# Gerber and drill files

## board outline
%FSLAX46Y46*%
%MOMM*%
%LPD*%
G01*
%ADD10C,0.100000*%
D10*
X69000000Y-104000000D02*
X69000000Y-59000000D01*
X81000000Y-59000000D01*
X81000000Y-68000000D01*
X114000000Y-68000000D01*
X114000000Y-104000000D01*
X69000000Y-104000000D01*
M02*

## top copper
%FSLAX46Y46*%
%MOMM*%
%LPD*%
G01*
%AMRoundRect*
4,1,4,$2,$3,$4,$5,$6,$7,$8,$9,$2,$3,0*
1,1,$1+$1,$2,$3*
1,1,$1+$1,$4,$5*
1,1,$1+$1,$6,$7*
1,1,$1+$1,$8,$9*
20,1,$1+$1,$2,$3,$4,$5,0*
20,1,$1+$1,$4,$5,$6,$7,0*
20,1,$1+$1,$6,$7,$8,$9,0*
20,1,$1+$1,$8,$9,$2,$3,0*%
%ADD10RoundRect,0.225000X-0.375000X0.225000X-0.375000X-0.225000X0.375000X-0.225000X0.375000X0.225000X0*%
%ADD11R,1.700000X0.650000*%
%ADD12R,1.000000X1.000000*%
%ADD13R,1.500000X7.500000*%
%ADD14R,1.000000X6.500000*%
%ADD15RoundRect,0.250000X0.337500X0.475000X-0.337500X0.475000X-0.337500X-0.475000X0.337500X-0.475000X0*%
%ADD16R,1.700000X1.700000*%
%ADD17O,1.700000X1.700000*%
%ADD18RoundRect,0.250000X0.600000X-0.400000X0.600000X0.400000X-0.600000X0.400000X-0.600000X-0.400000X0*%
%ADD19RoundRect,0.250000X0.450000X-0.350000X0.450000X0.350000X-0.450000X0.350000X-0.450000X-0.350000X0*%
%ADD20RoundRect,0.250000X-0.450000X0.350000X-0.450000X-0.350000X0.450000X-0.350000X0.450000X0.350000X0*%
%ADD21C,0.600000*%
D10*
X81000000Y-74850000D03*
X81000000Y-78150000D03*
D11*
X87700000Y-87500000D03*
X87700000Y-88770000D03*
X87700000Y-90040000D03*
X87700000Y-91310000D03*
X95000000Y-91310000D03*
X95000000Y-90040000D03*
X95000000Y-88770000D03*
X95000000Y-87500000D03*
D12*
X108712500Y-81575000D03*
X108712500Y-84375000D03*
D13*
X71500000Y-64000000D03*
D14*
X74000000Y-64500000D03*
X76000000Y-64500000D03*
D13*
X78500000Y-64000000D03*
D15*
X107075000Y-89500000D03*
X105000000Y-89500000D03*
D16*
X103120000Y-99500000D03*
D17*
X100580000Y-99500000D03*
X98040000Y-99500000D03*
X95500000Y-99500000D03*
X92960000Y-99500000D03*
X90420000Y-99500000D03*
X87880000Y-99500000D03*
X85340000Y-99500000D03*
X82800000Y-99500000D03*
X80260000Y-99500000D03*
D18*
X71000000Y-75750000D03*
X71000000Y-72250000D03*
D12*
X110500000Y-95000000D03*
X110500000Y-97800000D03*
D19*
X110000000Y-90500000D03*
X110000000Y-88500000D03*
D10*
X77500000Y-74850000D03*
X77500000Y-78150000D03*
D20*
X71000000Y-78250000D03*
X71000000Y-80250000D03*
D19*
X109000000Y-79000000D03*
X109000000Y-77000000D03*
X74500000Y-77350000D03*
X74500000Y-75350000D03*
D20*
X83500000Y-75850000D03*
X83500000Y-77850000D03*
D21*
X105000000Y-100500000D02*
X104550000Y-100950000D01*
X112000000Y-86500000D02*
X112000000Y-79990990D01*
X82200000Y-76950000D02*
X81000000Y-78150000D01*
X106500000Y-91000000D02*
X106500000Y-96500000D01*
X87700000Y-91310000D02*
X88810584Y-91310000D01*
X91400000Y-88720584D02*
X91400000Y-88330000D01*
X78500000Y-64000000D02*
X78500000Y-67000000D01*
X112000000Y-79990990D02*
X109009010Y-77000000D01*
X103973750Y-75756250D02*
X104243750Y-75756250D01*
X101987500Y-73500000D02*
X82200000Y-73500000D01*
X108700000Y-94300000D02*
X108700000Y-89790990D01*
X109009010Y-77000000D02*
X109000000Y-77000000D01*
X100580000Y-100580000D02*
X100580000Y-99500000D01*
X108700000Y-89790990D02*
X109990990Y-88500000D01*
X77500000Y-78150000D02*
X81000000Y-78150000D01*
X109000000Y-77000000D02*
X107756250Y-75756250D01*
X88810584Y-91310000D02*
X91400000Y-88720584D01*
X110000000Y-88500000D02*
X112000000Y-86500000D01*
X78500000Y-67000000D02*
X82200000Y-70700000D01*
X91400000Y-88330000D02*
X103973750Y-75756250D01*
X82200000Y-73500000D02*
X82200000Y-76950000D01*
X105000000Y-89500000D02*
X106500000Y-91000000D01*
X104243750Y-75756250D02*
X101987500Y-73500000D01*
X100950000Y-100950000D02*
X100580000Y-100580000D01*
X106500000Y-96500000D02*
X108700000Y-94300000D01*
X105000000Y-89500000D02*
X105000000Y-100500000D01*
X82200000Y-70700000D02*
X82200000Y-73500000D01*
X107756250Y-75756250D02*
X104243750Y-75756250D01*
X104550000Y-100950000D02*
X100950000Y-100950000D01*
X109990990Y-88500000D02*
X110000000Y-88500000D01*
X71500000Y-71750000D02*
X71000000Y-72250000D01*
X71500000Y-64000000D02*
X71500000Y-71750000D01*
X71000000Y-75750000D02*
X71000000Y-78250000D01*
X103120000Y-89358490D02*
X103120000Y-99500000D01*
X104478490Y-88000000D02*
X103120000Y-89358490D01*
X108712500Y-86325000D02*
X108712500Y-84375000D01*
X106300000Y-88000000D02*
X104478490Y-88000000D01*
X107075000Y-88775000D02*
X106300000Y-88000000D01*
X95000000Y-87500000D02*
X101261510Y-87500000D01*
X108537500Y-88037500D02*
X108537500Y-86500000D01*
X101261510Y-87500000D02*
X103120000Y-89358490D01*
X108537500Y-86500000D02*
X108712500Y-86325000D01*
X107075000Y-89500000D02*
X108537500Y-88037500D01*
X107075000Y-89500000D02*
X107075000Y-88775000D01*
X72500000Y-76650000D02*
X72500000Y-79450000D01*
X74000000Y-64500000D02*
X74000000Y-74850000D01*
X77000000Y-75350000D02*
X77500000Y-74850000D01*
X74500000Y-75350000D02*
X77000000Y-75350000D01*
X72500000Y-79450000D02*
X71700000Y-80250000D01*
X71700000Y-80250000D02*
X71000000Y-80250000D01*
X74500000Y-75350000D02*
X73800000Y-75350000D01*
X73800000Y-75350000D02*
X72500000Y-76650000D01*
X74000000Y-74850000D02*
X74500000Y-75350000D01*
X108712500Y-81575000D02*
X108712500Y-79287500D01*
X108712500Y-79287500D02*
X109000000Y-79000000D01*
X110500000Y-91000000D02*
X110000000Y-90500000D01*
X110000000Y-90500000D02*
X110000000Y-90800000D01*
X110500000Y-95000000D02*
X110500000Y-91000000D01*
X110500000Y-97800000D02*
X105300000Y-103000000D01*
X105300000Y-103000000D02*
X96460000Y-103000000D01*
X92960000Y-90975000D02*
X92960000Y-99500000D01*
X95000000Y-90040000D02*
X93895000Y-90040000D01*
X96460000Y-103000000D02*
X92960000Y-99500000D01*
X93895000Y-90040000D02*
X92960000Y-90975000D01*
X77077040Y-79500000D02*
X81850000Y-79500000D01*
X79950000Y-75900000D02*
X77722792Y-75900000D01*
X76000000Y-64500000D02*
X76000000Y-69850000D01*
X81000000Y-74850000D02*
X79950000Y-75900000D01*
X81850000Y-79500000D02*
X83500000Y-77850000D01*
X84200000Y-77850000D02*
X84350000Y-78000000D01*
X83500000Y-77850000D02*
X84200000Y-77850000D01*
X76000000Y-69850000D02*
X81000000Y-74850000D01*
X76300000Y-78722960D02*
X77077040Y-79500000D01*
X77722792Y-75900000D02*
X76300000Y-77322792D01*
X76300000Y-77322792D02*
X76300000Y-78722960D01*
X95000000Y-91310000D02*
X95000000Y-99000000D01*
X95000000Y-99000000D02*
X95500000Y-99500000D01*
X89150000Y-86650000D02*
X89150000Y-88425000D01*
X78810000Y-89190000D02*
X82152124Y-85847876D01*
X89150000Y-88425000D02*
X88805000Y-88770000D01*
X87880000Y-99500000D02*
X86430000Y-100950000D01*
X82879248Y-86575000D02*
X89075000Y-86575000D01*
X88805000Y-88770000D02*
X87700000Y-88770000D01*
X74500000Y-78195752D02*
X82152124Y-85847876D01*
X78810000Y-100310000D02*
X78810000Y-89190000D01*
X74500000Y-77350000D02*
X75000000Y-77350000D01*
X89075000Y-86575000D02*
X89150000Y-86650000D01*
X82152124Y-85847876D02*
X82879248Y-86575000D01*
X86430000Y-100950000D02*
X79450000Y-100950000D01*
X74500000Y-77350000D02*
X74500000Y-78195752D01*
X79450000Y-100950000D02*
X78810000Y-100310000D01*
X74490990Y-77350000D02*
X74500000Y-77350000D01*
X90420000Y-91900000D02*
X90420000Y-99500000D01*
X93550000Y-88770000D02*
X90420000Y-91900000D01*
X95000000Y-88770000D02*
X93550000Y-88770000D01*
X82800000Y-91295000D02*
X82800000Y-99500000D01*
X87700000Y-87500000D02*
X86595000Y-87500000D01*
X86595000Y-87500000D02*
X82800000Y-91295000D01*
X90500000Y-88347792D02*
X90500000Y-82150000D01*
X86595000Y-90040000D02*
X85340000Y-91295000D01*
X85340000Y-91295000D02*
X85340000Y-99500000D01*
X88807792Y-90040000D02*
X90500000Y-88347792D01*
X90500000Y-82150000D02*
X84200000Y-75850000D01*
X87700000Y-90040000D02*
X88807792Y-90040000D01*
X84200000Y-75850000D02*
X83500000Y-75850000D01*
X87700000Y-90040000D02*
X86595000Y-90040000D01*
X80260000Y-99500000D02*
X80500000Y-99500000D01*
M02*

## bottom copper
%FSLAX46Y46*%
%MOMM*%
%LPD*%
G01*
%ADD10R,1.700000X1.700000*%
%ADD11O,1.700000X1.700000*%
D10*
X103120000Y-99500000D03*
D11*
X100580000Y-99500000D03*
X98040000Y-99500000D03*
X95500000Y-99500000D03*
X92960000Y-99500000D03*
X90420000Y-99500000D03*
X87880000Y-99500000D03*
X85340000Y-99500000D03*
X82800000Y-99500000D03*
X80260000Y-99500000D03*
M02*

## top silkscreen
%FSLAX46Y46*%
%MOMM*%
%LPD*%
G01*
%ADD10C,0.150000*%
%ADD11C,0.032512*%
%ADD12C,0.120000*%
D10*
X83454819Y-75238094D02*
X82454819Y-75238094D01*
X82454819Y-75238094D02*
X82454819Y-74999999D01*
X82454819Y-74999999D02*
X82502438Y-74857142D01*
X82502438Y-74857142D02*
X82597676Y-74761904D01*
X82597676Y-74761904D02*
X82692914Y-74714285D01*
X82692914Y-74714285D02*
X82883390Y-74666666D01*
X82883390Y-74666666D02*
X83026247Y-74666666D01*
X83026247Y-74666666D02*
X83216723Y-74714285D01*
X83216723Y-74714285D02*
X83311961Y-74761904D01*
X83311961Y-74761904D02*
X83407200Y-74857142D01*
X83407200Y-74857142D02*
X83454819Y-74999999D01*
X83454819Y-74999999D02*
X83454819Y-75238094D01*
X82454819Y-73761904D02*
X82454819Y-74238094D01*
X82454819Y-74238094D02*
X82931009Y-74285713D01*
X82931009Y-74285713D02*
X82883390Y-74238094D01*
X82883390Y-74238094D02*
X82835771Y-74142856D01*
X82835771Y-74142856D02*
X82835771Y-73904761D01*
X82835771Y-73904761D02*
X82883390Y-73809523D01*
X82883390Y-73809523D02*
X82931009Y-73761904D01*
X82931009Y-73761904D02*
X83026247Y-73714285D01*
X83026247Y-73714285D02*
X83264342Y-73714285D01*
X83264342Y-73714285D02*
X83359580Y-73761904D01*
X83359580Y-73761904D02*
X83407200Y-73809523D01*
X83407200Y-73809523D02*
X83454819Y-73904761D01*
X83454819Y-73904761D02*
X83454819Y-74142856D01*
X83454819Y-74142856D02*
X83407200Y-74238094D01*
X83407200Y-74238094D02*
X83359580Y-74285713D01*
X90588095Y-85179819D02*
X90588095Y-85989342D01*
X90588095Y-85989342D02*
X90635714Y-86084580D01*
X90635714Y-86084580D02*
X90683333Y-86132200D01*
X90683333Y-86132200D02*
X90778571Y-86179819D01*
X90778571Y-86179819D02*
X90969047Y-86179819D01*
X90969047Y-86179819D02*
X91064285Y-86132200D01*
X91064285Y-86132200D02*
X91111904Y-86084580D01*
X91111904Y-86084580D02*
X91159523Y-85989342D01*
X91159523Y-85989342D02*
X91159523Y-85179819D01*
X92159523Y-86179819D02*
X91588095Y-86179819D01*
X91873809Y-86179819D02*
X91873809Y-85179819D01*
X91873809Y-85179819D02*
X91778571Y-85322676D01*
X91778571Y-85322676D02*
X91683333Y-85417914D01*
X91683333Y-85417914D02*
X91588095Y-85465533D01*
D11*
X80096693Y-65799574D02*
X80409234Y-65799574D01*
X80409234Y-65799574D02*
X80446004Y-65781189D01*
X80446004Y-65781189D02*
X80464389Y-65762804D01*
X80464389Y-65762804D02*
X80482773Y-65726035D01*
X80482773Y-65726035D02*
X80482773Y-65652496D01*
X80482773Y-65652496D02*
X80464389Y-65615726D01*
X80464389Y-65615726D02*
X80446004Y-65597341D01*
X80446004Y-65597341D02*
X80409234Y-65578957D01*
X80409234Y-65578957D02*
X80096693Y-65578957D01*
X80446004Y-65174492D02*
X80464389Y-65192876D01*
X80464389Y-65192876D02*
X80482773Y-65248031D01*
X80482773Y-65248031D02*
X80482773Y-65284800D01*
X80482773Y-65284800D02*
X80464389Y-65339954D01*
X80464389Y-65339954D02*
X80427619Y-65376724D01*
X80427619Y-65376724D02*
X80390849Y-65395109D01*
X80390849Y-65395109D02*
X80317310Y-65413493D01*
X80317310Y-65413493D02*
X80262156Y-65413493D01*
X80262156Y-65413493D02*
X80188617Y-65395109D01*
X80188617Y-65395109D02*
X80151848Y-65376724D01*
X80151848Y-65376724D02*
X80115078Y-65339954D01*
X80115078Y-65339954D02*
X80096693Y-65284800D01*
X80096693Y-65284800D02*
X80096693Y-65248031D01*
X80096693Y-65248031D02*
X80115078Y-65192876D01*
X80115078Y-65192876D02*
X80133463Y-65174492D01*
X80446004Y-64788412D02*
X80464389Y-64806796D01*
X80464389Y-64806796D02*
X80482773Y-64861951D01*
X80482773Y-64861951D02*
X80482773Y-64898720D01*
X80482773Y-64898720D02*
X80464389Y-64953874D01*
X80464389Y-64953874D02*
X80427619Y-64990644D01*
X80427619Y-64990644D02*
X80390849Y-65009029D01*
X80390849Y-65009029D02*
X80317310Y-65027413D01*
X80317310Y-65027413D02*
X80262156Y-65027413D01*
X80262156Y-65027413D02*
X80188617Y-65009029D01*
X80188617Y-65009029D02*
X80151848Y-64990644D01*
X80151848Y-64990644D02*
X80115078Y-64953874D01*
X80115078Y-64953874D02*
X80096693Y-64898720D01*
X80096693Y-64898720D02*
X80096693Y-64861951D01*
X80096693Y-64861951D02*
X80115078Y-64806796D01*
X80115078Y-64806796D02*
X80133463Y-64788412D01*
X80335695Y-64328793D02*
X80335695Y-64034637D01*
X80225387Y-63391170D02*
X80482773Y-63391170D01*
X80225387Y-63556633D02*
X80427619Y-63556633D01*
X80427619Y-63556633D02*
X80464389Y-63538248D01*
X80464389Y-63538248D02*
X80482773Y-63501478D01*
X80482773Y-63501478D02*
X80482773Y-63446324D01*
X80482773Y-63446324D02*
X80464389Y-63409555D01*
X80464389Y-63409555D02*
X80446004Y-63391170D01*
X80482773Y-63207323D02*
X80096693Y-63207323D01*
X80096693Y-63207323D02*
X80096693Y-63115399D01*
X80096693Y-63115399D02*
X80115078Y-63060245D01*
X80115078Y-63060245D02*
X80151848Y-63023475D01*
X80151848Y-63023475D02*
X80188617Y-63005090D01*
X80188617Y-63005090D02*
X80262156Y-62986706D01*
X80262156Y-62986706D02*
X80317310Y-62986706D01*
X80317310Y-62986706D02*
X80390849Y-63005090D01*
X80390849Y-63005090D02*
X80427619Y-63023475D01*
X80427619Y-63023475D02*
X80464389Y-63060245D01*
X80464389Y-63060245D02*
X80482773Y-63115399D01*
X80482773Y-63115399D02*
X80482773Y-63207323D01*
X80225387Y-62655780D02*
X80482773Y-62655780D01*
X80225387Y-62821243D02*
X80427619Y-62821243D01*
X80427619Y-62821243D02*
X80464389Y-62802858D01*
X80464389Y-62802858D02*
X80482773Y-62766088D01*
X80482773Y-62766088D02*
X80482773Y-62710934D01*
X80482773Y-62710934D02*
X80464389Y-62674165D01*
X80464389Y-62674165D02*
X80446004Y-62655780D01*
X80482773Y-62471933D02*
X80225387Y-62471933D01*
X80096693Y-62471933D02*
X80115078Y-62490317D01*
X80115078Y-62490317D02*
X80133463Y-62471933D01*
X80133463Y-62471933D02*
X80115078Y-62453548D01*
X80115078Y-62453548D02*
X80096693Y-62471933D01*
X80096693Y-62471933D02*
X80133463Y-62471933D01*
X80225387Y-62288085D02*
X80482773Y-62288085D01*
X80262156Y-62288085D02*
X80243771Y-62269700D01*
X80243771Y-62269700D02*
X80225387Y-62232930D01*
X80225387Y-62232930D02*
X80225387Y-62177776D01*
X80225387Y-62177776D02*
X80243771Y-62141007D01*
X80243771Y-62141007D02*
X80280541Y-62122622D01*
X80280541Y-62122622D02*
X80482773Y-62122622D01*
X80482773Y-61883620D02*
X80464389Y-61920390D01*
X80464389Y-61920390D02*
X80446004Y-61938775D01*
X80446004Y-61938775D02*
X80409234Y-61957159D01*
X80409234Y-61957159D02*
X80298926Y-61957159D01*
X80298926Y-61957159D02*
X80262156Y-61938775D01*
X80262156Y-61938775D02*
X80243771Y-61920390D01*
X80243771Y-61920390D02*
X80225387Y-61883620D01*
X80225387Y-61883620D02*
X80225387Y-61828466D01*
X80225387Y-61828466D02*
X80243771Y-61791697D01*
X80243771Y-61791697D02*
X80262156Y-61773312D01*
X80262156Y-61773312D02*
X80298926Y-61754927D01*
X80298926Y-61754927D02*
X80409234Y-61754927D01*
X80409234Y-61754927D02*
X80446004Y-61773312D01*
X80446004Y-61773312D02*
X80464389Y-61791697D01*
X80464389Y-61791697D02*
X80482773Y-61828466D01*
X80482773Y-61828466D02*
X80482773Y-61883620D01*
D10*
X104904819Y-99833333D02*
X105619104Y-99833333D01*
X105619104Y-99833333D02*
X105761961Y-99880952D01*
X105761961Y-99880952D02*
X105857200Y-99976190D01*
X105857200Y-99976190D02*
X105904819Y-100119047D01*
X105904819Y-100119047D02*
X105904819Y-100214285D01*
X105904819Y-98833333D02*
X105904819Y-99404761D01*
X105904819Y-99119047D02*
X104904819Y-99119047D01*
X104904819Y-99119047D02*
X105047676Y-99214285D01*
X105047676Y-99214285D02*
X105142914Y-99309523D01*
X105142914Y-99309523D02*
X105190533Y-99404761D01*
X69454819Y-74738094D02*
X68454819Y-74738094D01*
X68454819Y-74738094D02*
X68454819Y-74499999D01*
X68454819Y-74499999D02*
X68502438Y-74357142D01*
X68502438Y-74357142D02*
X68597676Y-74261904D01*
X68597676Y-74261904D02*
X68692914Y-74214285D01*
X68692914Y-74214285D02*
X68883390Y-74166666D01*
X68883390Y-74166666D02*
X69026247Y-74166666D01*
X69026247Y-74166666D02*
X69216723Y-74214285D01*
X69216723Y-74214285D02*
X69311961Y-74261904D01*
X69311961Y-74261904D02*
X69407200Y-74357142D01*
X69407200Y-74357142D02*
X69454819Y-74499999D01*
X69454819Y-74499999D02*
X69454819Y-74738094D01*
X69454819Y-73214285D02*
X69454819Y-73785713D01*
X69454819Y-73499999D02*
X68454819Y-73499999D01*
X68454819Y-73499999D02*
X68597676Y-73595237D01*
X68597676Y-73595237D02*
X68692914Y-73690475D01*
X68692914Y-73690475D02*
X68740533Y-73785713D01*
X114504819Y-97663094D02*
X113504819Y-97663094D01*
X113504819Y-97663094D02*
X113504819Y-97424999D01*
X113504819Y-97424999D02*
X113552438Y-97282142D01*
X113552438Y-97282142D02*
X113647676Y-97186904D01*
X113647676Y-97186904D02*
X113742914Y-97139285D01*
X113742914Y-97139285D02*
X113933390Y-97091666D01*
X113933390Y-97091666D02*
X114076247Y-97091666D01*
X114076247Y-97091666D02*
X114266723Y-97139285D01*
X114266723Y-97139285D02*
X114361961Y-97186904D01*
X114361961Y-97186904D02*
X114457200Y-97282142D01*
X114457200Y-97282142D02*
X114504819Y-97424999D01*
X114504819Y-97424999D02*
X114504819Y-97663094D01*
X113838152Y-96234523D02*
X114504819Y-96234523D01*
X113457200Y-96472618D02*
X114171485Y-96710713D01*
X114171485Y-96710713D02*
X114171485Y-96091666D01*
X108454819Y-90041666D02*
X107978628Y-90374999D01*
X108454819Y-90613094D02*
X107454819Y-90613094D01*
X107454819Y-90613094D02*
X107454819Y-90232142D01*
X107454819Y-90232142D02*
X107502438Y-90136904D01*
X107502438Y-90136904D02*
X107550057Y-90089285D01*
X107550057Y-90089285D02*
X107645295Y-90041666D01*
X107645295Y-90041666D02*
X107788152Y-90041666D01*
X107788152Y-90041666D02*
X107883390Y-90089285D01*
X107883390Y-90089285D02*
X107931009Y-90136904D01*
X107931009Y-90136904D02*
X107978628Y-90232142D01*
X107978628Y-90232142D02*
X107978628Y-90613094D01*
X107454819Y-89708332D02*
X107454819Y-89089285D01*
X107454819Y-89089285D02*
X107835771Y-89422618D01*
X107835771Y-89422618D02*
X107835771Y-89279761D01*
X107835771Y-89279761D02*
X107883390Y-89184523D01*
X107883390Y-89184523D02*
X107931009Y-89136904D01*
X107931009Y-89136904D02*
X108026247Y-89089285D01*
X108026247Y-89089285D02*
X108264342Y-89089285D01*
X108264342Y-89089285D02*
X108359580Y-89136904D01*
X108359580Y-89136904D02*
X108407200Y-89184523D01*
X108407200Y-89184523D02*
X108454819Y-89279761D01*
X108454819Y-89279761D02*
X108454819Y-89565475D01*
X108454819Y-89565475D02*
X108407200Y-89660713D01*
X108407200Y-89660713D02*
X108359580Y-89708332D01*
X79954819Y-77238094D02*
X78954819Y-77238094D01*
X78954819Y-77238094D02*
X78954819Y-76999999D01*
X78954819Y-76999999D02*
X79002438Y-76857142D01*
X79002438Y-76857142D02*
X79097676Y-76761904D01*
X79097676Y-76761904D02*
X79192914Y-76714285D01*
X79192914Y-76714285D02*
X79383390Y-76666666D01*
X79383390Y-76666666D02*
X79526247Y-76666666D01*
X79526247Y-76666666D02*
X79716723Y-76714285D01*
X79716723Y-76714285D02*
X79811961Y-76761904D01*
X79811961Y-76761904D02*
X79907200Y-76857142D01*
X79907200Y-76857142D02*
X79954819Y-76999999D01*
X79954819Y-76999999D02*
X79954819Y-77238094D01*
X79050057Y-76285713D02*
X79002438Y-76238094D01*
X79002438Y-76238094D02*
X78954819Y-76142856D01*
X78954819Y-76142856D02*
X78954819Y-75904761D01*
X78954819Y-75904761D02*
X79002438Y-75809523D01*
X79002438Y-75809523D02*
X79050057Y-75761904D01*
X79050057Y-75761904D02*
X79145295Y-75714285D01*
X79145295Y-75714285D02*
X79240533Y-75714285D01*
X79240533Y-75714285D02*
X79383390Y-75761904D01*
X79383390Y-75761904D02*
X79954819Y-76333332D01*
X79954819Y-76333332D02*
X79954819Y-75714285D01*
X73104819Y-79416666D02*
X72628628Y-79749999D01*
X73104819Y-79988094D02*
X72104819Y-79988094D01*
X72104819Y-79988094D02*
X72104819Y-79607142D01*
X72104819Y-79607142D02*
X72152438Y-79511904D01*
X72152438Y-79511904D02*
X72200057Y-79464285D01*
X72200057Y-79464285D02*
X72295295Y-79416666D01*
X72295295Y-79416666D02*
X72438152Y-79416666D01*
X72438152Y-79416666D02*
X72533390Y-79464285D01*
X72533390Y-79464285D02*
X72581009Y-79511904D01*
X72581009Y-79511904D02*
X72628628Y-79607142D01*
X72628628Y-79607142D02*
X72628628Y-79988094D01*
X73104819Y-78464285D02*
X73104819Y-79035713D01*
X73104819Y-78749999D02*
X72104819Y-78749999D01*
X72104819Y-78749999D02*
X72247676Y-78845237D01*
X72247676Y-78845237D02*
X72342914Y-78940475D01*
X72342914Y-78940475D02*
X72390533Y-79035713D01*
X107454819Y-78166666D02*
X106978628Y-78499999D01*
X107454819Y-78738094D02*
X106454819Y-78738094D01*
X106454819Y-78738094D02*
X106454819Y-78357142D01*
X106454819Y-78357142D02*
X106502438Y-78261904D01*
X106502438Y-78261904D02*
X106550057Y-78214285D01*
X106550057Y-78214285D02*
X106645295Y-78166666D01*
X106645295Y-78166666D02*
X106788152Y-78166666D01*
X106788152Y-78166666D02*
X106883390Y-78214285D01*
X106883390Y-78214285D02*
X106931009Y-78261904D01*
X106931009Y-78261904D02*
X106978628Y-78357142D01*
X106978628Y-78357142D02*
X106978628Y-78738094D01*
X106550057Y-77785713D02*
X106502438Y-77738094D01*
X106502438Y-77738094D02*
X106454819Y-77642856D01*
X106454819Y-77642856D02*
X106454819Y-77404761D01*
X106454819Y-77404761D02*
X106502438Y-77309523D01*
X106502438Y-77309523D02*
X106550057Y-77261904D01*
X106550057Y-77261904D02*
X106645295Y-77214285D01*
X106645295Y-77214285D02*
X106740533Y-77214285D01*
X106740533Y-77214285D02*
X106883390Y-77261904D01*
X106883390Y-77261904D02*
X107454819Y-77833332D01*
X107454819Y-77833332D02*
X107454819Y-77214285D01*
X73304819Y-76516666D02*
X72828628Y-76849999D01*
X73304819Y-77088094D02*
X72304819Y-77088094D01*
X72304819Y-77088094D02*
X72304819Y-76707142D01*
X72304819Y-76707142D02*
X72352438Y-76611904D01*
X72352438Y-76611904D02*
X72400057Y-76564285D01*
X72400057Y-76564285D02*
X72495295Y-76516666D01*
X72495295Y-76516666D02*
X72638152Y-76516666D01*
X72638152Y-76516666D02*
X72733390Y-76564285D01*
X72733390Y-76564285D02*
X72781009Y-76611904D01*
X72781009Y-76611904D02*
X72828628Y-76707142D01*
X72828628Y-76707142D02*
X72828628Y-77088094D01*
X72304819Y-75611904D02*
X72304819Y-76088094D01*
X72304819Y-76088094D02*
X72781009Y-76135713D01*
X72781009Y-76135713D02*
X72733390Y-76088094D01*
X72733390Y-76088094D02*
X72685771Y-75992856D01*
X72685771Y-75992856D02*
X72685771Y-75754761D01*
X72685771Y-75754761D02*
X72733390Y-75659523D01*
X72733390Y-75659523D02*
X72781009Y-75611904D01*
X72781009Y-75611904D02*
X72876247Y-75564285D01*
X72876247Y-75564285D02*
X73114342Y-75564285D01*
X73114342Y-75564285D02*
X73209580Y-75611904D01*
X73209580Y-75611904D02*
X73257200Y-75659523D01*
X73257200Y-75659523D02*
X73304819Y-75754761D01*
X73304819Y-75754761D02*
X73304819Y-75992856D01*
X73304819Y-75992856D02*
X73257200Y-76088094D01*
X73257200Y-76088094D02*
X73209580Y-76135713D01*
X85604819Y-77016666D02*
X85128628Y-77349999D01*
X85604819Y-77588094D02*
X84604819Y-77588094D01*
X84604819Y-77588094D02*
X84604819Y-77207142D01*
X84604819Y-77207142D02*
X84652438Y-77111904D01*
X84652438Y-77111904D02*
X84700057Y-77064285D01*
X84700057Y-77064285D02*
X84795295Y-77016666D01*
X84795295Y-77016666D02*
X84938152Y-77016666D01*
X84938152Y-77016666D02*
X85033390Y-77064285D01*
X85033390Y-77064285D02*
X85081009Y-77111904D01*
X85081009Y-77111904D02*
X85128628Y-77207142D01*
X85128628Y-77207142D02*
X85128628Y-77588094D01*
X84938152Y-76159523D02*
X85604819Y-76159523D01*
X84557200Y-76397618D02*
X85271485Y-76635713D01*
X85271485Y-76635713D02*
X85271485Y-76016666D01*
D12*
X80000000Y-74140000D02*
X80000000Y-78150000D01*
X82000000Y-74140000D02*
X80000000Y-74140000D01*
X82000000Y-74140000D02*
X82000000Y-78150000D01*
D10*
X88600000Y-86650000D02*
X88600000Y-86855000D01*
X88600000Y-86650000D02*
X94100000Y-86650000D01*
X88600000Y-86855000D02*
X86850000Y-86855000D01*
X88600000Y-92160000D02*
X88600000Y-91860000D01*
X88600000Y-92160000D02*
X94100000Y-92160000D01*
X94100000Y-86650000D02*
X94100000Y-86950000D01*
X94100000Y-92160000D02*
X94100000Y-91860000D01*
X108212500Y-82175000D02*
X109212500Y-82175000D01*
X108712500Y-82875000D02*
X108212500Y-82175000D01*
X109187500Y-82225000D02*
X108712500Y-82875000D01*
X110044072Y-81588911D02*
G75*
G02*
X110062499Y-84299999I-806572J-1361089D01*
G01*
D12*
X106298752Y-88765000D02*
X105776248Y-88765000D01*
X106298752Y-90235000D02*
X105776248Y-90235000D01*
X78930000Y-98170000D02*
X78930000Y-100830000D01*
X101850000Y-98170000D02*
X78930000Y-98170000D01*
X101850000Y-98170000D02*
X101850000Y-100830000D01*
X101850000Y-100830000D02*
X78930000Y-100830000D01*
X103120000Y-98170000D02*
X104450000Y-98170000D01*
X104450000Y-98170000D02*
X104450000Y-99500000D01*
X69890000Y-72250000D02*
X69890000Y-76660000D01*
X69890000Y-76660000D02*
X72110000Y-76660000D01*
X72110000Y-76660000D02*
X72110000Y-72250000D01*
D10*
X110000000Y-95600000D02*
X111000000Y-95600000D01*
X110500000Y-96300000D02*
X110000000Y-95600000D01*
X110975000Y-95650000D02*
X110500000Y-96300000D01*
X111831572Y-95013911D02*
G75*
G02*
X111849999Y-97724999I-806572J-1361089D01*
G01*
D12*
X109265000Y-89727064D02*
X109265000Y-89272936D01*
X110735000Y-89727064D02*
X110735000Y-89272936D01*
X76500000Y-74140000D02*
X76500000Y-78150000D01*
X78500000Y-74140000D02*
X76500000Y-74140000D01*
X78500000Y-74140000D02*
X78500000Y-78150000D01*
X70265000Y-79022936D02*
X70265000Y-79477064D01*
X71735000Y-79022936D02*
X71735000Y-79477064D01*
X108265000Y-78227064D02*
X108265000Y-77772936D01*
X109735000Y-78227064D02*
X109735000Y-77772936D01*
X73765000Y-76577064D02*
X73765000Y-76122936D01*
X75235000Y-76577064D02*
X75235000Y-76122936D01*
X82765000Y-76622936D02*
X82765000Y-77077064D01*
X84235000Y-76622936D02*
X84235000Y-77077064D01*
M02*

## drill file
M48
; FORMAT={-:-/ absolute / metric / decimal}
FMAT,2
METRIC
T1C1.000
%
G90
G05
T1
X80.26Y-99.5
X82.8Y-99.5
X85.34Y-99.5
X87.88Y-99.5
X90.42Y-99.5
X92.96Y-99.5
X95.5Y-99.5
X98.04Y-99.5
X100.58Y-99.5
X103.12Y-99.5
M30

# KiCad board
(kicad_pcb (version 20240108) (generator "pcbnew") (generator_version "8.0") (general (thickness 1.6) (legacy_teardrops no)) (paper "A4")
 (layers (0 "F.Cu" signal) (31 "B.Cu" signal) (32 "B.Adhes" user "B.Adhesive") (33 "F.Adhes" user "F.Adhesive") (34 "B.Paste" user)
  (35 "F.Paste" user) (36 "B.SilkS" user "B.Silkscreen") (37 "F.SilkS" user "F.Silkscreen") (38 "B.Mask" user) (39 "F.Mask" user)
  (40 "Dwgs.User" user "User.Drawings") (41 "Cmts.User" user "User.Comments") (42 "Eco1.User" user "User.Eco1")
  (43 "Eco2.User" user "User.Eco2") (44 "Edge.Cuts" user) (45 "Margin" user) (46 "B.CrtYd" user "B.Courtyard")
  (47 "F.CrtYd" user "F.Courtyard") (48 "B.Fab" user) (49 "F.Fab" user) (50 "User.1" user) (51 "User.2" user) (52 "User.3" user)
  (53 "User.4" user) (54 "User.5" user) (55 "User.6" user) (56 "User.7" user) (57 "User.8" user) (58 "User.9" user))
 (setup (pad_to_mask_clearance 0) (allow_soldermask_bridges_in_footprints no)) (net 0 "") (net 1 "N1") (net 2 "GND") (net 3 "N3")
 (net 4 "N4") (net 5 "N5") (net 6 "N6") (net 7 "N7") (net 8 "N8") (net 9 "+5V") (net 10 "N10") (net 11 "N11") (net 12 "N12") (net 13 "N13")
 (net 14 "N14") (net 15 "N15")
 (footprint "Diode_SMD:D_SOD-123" (layer "F.Cu") (at 81 76.5 -90)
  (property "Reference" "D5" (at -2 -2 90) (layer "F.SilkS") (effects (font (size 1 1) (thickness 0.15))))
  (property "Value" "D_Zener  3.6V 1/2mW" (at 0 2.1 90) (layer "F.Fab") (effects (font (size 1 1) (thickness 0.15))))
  (fp_line (start -2.36 1) (end 1.65 1) (stroke (width 0.12) (type solid)) (layer "F.SilkS"))
  (fp_line (start -2.36 -1) (end -2.36 1) (stroke (width 0.12) (type solid)) (layer "F.SilkS"))
  (fp_line (start -2.36 -1) (end 1.65 -1) (stroke (width 0.12) (type solid)) (layer "F.SilkS"))
  (pad "1" smd roundrect (at -1.65 0 270) (size 0.9 1.2) (layers "F.Cu" "F.Paste" "F.Mask") (roundrect_rratio 0.25) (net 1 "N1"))
  (pad "2" smd roundrect (at 1.65 0 270) (size 0.9 1.2) (layers "F.Cu" "F.Paste" "F.Mask") (roundrect_rratio 0.25) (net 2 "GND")))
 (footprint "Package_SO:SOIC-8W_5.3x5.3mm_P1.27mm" (layer "F.Cu") (at 91.35 89.405)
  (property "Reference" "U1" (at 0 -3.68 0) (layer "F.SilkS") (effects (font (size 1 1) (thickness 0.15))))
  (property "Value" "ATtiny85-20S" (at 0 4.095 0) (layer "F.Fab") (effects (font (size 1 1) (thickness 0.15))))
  (fp_line (start -2.75 -2.755) (end -2.75 -2.55) (stroke (width 0.15) (type solid)) (layer "F.SilkS"))
  (fp_line (start -2.75 -2.755) (end 2.75 -2.755) (stroke (width 0.15) (type solid)) (layer "F.SilkS"))
  (fp_line (start -2.75 -2.55) (end -4.5 -2.55) (stroke (width 0.15) (type solid)) (layer "F.SilkS"))
  (fp_line (start -2.75 2.755) (end -2.75 2.455) (stroke (width 0.15) (type solid)) (layer "F.SilkS"))
  (fp_line (start -2.75 2.755) (end 2.75 2.755) (stroke (width 0.15) (type solid)) (layer "F.SilkS"))
  (fp_line (start 2.75 -2.755) (end 2.75 -2.455) (stroke (width 0.15) (type solid)) (layer "F.SilkS"))
  (fp_line (start 2.75 2.755) (end 2.75 2.455) (stroke (width 0.15) (type solid)) (layer "F.SilkS"))
  (pad "1" smd rect (at -3.65 -1.905) (size 1.7 0.65) (layers "F.Cu" "F.Paste" "F.Mask") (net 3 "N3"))
  (pad "2" smd rect (at -3.65 -0.635) (size 1.7 0.65) (layers "F.Cu" "F.Paste" "F.Mask") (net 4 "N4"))
  (pad "3" smd rect (at -3.65 0.635) (size 1.7 0.65) (layers "F.Cu" "F.Paste" "F.Mask") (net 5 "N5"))
  (pad "4" smd rect (at -3.65 1.905) (size 1.7 0.65) (layers "F.Cu" "F.Paste" "F.Mask") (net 2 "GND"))
  (pad "5" smd rect (at 3.65 1.905) (size 1.7 0.65) (layers "F.Cu" "F.Paste" "F.Mask") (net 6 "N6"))
  (pad "6" smd rect (at 3.65 0.635) (size 1.7 0.65) (layers "F.Cu" "F.Paste" "F.Mask") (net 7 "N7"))
  (pad "7" smd rect (at 3.65 -0.635) (size 1.7 0.65) (layers "F.Cu" "F.Paste" "F.Mask") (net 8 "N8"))
  (pad "8" smd rect (at 3.65 -1.905) (size 1.7 0.65) (layers "F.Cu" "F.Paste" "F.Mask") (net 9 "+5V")))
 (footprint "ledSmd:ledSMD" (layer "F.Cu") (at 108.7125 83.375 -90)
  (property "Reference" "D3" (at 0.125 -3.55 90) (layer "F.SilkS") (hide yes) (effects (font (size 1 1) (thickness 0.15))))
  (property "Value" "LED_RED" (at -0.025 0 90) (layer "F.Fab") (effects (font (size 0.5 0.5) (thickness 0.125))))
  (fp_line (start -1.2 0.5) (end -1.2 -0.5) (stroke (width 0.15) (type solid)) (layer "F.SilkS"))
  (fp_line (start -0.5 0) (end -1.2 0.5) (stroke (width 0.15) (type solid)) (layer "F.SilkS"))
  (fp_line (start -1.15 -0.475) (end -0.5 0) (stroke (width 0.15) (type solid)) (layer "F.SilkS"))
  (fp_arc (start -1.786089 -1.331572) (mid -0.435753 -2.107089) (end 0.924999 -1.349999) (stroke (width 0.15) (type solid))
   (layer "F.SilkS"))
  (pad "1" smd rect (at -1.8 0 270) (size 1 1) (layers "F.Cu" "F.Paste" "F.Mask") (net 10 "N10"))
  (pad "2" smd rect (at 1 0 270) (size 1 1) (layers "F.Cu" "F.Paste" "F.Mask") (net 9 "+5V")))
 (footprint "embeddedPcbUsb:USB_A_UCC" (layer "F.Cu") (at 75 64.2 -90)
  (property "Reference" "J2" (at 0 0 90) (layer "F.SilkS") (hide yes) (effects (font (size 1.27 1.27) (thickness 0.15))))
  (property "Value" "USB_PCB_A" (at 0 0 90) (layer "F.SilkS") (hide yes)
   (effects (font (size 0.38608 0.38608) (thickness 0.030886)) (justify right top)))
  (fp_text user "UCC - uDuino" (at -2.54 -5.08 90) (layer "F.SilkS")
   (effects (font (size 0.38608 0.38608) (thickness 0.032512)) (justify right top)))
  (pad "1" smd rect (at -0.2 3.5 270) (size 7.5 1.5) (layers "F.Cu" "F.Paste" "F.Mask") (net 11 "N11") (solder_mask_margin 0.1016))
  (pad "2" smd rect (at 0.3 1 270) (size 6.5 1) (layers "F.Cu" "F.Paste" "F.Mask") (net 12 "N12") (solder_mask_margin 0.1016))
  (pad "3" smd rect (at 0.3 -1 270) (size 6.5 1) (layers "F.Cu" "F.Paste" "F.Mask") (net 1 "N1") (solder_mask_margin 0.1016))
  (pad "4" smd rect (at -0.2 -3.5 270) (size 7.5 1.5) (layers "F.Cu" "F.Paste" "F.Mask") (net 2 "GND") (solder_mask_margin 0.1016)))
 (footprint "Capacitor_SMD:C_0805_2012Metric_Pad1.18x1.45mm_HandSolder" (layer "F.Cu") (at 106.0375 89.5 180)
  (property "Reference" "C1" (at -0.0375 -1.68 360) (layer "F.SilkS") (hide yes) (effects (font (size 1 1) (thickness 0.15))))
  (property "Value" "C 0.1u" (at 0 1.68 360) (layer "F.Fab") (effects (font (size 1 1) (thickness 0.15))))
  (fp_line (start -0.261252 0.735) (end 0.261252 0.735) (stroke (width 0.12) (type solid)) (layer "F.SilkS"))
  (fp_line (start -0.261252 -0.735) (end 0.261252 -0.735) (stroke (width 0.12) (type solid)) (layer "F.SilkS"))
  (pad "1" smd roundrect (at -1.0375 0 180) (size 1.175 1.45) (layers "F.Cu" "F.Paste" "F.Mask") (roundrect_rratio 0.212766) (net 9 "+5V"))
  (pad "2" smd roundrect (at 1.0375 0 180) (size 1.175 1.45) (layers "F.Cu" "F.Paste" "F.Mask") (roundrect_rratio 0.212766) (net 2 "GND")))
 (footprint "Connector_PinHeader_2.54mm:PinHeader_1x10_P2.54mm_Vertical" (layer "F.Cu") (at 103.12 99.5 -90)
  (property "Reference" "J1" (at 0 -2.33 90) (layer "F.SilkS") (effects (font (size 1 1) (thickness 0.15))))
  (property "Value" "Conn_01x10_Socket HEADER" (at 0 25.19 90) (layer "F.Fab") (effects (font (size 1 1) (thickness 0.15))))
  (fp_line (start -1.33 24.19) (end 1.33 24.19) (stroke (width 0.12) (type solid)) (layer "F.SilkS"))
  (fp_line (start -1.33 1.27) (end -1.33 24.19) (stroke (width 0.12) (type solid)) (layer "F.SilkS"))
  (fp_line (start -1.33 1.27) (end 1.33 1.27) (stroke (width 0.12) (type solid)) (layer "F.SilkS"))
  (fp_line (start 1.33 1.27) (end 1.33 24.19) (stroke (width 0.12) (type solid)) (layer "F.SilkS"))
  (fp_line (start -1.33 0) (end -1.33 -1.33) (stroke (width 0.12) (type solid)) (layer "F.SilkS"))
  (fp_line (start -1.33 -1.33) (end 0 -1.33) (stroke (width 0.12) (type solid)) (layer "F.SilkS"))
  (pad "1" thru_hole rect (at 0 0 270) (size 1.7 1.7) (drill 1) (layers "*.Cu" "*.Mask") (remove_unused_layers no) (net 9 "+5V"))
  (pad "2" thru_hole oval (at 0 2.54 270) (size 1.7 1.7) (drill 1) (layers "*.Cu" "*.Mask") (remove_unused_layers no) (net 2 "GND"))
  (pad "3" thru_hole oval (at 0 5.08 270) (size 1.7 1.7) (drill 1) (layers "*.Cu" "*.Mask") (remove_unused_layers no) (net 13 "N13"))
  (pad "4" thru_hole oval (at 0 7.62 270) (size 1.7 1.7) (drill 1) (layers "*.Cu" "*.Mask") (remove_unused_layers no) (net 6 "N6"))
  (pad "5" thru_hole oval (at 0 10.16 270) (size 1.7 1.7) (drill 1) (layers "*.Cu" "*.Mask") (remove_unused_layers no) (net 7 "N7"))
  (pad "6" thru_hole oval (at 0 12.7 270) (size 1.7 1.7) (drill 1) (layers "*.Cu" "*.Mask") (remove_unused_layers no) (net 8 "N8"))
  (pad "7" thru_hole oval (at 0 15.24 270) (size 1.7 1.7) (drill 1) (layers "*.Cu" "*.Mask") (remove_unused_layers no) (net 4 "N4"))
  (pad "8" thru_hole oval (at 0 17.78 270) (size 1.7 1.7) (drill 1) (layers "*.Cu" "*.Mask") (remove_unused_layers no) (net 5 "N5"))
  (pad "9" thru_hole oval (at 0 20.32 270) (size 1.7 1.7) (drill 1) (layers "*.Cu" "*.Mask") (remove_unused_layers no) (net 3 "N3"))
  (pad "10" thru_hole oval (at 0 22.86 270) (size 1.7 1.7) (drill 1) (layers "*.Cu" "*.Mask") (remove_unused_layers no) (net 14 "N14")))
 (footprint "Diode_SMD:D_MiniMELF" (layer "F.Cu") (at 71 74 90)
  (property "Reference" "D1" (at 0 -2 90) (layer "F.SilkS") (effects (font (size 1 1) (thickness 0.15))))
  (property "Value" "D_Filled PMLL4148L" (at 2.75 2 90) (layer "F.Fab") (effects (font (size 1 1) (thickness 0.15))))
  (fp_line (start 1.75 -1.11) (end -2.66 -1.11) (stroke (width 0.12) (type solid)) (layer "F.SilkS"))
  (fp_line (start -2.66 -1.11) (end -2.66 1.11) (stroke (width 0.12) (type solid)) (layer "F.SilkS"))
  (fp_line (start -2.66 1.11) (end 1.75 1.11) (stroke (width 0.12) (type solid)) (layer "F.SilkS"))
  (pad "1" smd roundrect (at -1.75 0 90) (size 1.3 1.7) (layers "F.Cu" "F.Paste" "F.Mask") (roundrect_rratio 0.1923076923) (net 9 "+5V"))
  (pad "2" smd roundrect (at 1.75 0 90) (size 1.3 1.7) (layers "F.Cu" "F.Paste" "F.Mask") (roundrect_rratio 0.1923076923) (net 11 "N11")))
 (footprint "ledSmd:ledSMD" (layer "F.Cu") (at 110.5 96.8 -90)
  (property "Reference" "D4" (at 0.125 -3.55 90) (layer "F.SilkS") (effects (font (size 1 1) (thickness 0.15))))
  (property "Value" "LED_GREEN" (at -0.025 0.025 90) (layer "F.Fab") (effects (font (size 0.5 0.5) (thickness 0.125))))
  (fp_line (start -1.2 0.5) (end -1.2 -0.5) (stroke (width 0.15) (type solid)) (layer "F.SilkS"))
  (fp_line (start -0.5 0) (end -1.2 0.5) (stroke (width 0.15) (type solid)) (layer "F.SilkS"))
  (fp_line (start -1.15 -0.475) (end -0.5 0) (stroke (width 0.15) (type solid)) (layer "F.SilkS"))
  (fp_arc (start -1.786089 -1.331572) (mid -0.435753 -2.107089) (end 0.924999 -1.349999) (stroke (width 0.15) (type solid))
   (layer "F.SilkS"))
  (pad "1" smd rect (at -1.8 0 270) (size 1 1) (layers "F.Cu" "F.Paste" "F.Mask") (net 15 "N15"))
  (pad "2" smd rect (at 1 0 270) (size 1 1) (layers "F.Cu" "F.Paste" "F.Mask") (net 7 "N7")))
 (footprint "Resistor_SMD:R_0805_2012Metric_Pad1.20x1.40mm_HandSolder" (layer "F.Cu") (at 110 89.5 90)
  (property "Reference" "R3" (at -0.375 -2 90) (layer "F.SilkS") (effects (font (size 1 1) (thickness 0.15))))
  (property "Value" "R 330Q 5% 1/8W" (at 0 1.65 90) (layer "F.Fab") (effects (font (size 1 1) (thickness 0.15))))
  (fp_line (start -0.227064 -0.735) (end 0.227064 -0.735) (stroke (width 0.12) (type solid)) (layer "F.SilkS"))
  (fp_line (start -0.227064 0.735) (end 0.227064 0.735) (stroke (width 0.12) (type solid)) (layer "F.SilkS"))
  (pad "1" smd roundrect (at -1 0 90) (size 1.2 1.4) (layers "F.Cu" "F.Paste" "F.Mask") (roundrect_rratio 0.208333) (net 15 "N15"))
  (pad "2" smd roundrect (at 1 0 90) (size 1.2 1.4) (layers "F.Cu" "F.Paste" "F.Mask") (roundrect_rratio 0.208333) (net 2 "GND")))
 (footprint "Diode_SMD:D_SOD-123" (layer "F.Cu") (at 77.5 76.5 -90)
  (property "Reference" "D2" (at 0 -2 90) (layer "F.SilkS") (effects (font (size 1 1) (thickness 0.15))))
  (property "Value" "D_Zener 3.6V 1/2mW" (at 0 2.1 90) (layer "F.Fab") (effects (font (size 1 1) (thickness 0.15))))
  (fp_line (start -2.36 1) (end 1.65 1) (stroke (width 0.12) (type solid)) (layer "F.SilkS"))
  (fp_line (start -2.36 -1) (end -2.36 1) (stroke (width 0.12) (type solid)) (layer "F.SilkS"))
  (fp_line (start -2.36 -1) (end 1.65 -1) (stroke (width 0.12) (type solid)) (layer "F.SilkS"))
  (pad "1" smd roundrect (at -1.65 0 270) (size 0.9 1.2) (layers "F.Cu" "F.Paste" "F.Mask") (roundrect_rratio 0.25) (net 12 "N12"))
  (pad "2" smd roundrect (at 1.65 0 270) (size 0.9 1.2) (layers "F.Cu" "F.Paste" "F.Mask") (roundrect_rratio 0.25) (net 2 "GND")))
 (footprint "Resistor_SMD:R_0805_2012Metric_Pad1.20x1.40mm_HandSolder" (layer "F.Cu") (at 71 79.25 -90)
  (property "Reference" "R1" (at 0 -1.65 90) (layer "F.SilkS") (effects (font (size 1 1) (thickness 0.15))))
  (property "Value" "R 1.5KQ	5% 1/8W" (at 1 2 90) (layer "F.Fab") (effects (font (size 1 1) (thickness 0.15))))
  (fp_line (start -0.227064 0.735) (end 0.227064 0.735) (stroke (width 0.12) (type solid)) (layer "F.SilkS"))
  (fp_line (start -0.227064 -0.735) (end 0.227064 -0.735) (stroke (width 0.12) (type solid)) (layer "F.SilkS"))
  (pad "1" smd roundrect (at -1 0 270) (size 1.2 1.4) (layers "F.Cu" "F.Paste" "F.Mask") (roundrect_rratio 0.208333) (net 9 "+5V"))
  (pad "2" smd roundrect (at 1 0 270) (size 1.2 1.4) (layers "F.Cu" "F.Paste" "F.Mask") (roundrect_rratio 0.208333) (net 12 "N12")))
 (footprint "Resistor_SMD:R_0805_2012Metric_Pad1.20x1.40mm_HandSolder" (layer "F.Cu") (at 109 78 90)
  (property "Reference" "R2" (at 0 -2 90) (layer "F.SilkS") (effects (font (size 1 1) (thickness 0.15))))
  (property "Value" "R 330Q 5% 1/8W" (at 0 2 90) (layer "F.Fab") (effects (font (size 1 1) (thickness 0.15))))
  (fp_line (start -0.227064 -0.735) (end 0.227064 -0.735) (stroke (width 0.12) (type solid)) (layer "F.SilkS"))
  (fp_line (start -0.227064 0.735) (end 0.227064 0.735) (stroke (width 0.12) (type solid)) (layer "F.SilkS"))
  (pad "1" smd roundrect (at -1 0 90) (size 1.2 1.4) (layers "F.Cu" "F.Paste" "F.Mask") (roundrect_rratio 0.208333) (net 10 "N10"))
  (pad "2" smd roundrect (at 1 0 90) (size 1.2 1.4) (layers "F.Cu" "F.Paste" "F.Mask") (roundrect_rratio 0.208333) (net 2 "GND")))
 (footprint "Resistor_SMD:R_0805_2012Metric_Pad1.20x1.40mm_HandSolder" (layer "F.Cu") (at 74.5 76.35 90)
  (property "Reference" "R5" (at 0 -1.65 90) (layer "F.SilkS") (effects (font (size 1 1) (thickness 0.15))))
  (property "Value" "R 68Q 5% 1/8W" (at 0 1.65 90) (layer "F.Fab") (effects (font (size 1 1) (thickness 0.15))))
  (fp_line (start -0.227064 -0.735) (end 0.227064 -0.735) (stroke (width 0.12) (type solid)) (layer "F.SilkS"))
  (fp_line (start -0.227064 0.735) (end 0.227064 0.735) (stroke (width 0.12) (type solid)) (layer "F.SilkS"))
  (pad "1" smd roundrect (at -1 0 90) (size 1.2 1.4) (layers "F.Cu" "F.Paste" "F.Mask") (roundrect_rratio 0.208333) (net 4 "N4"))
  (pad "2" smd roundrect (at 1 0 90) (size 1.2 1.4) (layers "F.Cu" "F.Paste" "F.Mask") (roundrect_rratio 0.208333) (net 12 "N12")))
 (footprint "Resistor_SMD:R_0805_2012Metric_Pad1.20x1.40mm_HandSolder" (layer "F.Cu") (at 83.5 76.85 -90)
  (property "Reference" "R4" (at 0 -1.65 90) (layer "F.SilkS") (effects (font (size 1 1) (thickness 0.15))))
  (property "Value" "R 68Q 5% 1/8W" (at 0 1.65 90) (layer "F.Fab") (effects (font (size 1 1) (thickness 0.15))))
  (fp_line (start -0.227064 0.735) (end 0.227064 0.735) (stroke (width 0.12) (type solid)) (layer "F.SilkS"))
  (fp_line (start -0.227064 -0.735) (end 0.227064 -0.735) (stroke (width 0.12) (type solid)) (layer "F.SilkS"))
  (pad "1" smd roundrect (at -1 0 270) (size 1.2 1.4) (layers "F.Cu" "F.Paste" "F.Mask") (roundrect_rratio 0.208333) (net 5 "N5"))
  (pad "2" smd roundrect (at 1 0 270) (size 1.2 1.4) (layers "F.Cu" "F.Paste" "F.Mask") (roundrect_rratio 0.208333) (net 1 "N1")))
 (gr_poly
  (pts (xy 69 104) (xy 69 59) (xy 81 59) (xy 81 68) (xy 114 68) (xy 114 104)) (stroke (width 0.1) (type solid)) (fill none)
  (layer "Edge.Cuts"))
 (segment (start 105 100.5) (end 104.55 100.95) (width 0.6) (layer "F.Cu") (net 2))
 (segment (start 112 86.5) (end 112 79.99099) (width 0.6) (layer "F.Cu") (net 2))
 (segment (start 82.2 76.95) (end 81 78.15) (width 0.6) (layer "F.Cu") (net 2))
 (segment (start 106.5 91) (end 106.5 96.5) (width 0.6) (layer "F.Cu") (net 2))
 (segment (start 87.7 91.31) (end 88.810584 91.31) (width 0.6) (layer "F.Cu") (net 2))
 (segment (start 91.4 88.720584) (end 91.4 88.33) (width 0.6) (layer "F.Cu") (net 2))
 (segment (start 78.5 64) (end 78.5 67) (width 0.6) (layer "F.Cu") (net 2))
 (segment (start 112 79.99099) (end 109.00901 77) (width 0.6) (layer "F.Cu") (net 2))
 (segment (start 103.97375 75.75625) (end 104.24375 75.75625) (width 0.6) (layer "F.Cu") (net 2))
 (segment (start 101.9875 73.5) (end 82.2 73.5) (width 0.6) (layer "F.Cu") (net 2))
 (segment (start 108.7 94.3) (end 108.7 89.79099) (width 0.6) (layer "F.Cu") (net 2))
 (segment (start 109.00901 77) (end 109 77) (width 0.6) (layer "F.Cu") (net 2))
 (segment (start 100.58 100.58) (end 100.58 99.5) (width 0.6) (layer "F.Cu") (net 2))
 (segment (start 108.7 89.79099) (end 109.99099 88.5) (width 0.6) (layer "F.Cu") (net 2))
 (segment (start 77.5 78.15) (end 81 78.15) (width 0.6) (layer "F.Cu") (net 2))
 (segment (start 109 77) (end 107.75625 75.75625) (width 0.6) (layer "F.Cu") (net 2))
 (segment (start 88.810584 91.31) (end 91.4 88.720584) (width 0.6) (layer "F.Cu") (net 2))
 (segment (start 110 88.5) (end 112 86.5) (width 0.6) (layer "F.Cu") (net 2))
 (segment (start 78.5 67) (end 82.2 70.7) (width 0.6) (layer "F.Cu") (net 2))
 (segment (start 91.4 88.33) (end 103.97375 75.75625) (width 0.6) (layer "F.Cu") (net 2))
 (segment (start 82.2 73.5) (end 82.2 76.95) (width 0.6) (layer "F.Cu") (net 2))
 (segment (start 105 89.5) (end 106.5 91) (width 0.6) (layer "F.Cu") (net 2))
 (segment (start 104.24375 75.75625) (end 101.9875 73.5) (width 0.6) (layer "F.Cu") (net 2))
 (segment (start 100.95 100.95) (end 100.58 100.58) (width 0.6) (layer "F.Cu") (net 2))
 (segment (start 106.5 96.5) (end 108.7 94.3) (width 0.6) (layer "F.Cu") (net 2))
 (segment (start 105 89.5) (end 105 100.5) (width 0.6) (layer "F.Cu") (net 2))
 (segment (start 82.2 70.7) (end 82.2 73.5) (width 0.6) (layer "F.Cu") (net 2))
 (segment (start 107.75625 75.75625) (end 104.24375 75.75625) (width 0.6) (layer "F.Cu") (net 2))
 (segment (start 104.55 100.95) (end 100.95 100.95) (width 0.6) (layer "F.Cu") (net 2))
 (segment (start 109.99099 88.5) (end 110 88.5) (width 0.6) (layer "F.Cu") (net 2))
 (segment (start 71.5 71.75) (end 71 72.25) (width 0.6) (layer "F.Cu") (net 11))
 (segment (start 71.5 64) (end 71.5 71.75) (width 0.6) (layer "F.Cu") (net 11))
 (segment (start 71 75.75) (end 71 78.25) (width 0.6) (layer "F.Cu") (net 9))
 (segment (start 103.12 89.35849) (end 103.12 99.5) (width 0.6) (layer "F.Cu") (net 9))
 (segment (start 104.47849 88) (end 103.12 89.35849) (width 0.6) (layer "F.Cu") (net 9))
 (segment (start 108.7125 86.325) (end 108.7125 84.375) (width 0.6) (layer "F.Cu") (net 9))
 (segment (start 106.3 88) (end 104.47849 88) (width 0.6) (layer "F.Cu") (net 9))
 (segment (start 107.075 88.775) (end 106.3 88) (width 0.6) (layer "F.Cu") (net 9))
 (segment (start 95 87.5) (end 101.26151 87.5) (width 0.6) (layer "F.Cu") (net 9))
 (segment (start 108.5375 88.0375) (end 108.5375 86.5) (width 0.6) (layer "F.Cu") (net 9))
 (segment (start 101.26151 87.5) (end 103.12 89.35849) (width 0.6) (layer "F.Cu") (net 9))
 (segment (start 108.5375 86.5) (end 108.7125 86.325) (width 0.6) (layer "F.Cu") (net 9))
 (segment (start 107.075 89.5) (end 108.5375 88.0375) (width 0.6) (layer "F.Cu") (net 9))
 (segment (start 107.075 89.5) (end 107.075 88.775) (width 0.6) (layer "F.Cu") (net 9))
 (segment (start 72.5 76.65) (end 72.5 79.45) (width 0.6) (layer "F.Cu") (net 12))
 (segment (start 74 64.5) (end 74 74.85) (width 0.6) (layer "F.Cu") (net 12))
 (segment (start 77 75.35) (end 77.5 74.85) (width 0.6) (layer "F.Cu") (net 12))
 (segment (start 74.5 75.35) (end 77 75.35) (width 0.6) (layer "F.Cu") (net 12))
 (segment (start 72.5 79.45) (end 71.7 80.25) (width 0.6) (layer "F.Cu") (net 12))
 (segment (start 71.7 80.25) (end 71 80.25) (width 0.6) (layer "F.Cu") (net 12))
 (segment (start 74.5 75.35) (end 73.8 75.35) (width 0.6) (layer "F.Cu") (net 12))
 (segment (start 73.8 75.35) (end 72.5 76.65) (width 0.6) (layer "F.Cu") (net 12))
 (segment (start 74 74.85) (end 74.5 75.35) (width 0.6) (layer "F.Cu") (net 12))
 (segment (start 108.7125 81.575) (end 108.7125 79.2875) (width 0.6) (layer "F.Cu") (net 10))
 (segment (start 108.7125 79.2875) (end 109 79) (width 0.6) (layer "F.Cu") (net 10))
 (segment (start 110.5 91) (end 110 90.5) (width 0.6) (layer "F.Cu") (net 15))
 (segment (start 110 90.5) (end 110 90.8) (width 0.6) (layer "F.Cu") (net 15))
 (segment (start 110.5 95) (end 110.5 91) (width 0.6) (layer "F.Cu") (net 15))
 (segment (start 110.5 97.8) (end 105.3 103) (width 0.6) (layer "F.Cu") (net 7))
 (segment (start 105.3 103) (end 96.46 103) (width 0.6) (layer "F.Cu") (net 7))
 (segment (start 92.96 90.975) (end 92.96 99.5) (width 0.6) (layer "F.Cu") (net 7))
 (segment (start 95 90.04) (end 93.895 90.04) (width 0.6) (layer "F.Cu") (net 7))
 (segment (start 96.46 103) (end 92.96 99.5) (width 0.6) (layer "F.Cu") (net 7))
 (segment (start 93.895 90.04) (end 92.96 90.975) (width 0.6) (layer "F.Cu") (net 7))
 (segment (start 77.07704 79.5) (end 81.85 79.5) (width 0.6) (layer "F.Cu") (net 1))
 (segment (start 79.95 75.9) (end 77.722792 75.9) (width 0.6) (layer "F.Cu") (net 1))
 (segment (start 76 64.5) (end 76 69.85) (width 0.6) (layer "F.Cu") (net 1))
 (segment (start 81 74.85) (end 79.95 75.9) (width 0.6) (layer "F.Cu") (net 1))
 (segment (start 81.85 79.5) (end 83.5 77.85) (width 0.6) (layer "F.Cu") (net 1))
 (segment (start 84.2 77.85) (end 84.35 78) (width 0.6) (layer "F.Cu") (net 1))
 (segment (start 83.5 77.85) (end 84.2 77.85) (width 0.6) (layer "F.Cu") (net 1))
 (segment (start 76 69.85) (end 81 74.85) (width 0.6) (layer "F.Cu") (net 1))
 (segment (start 76.3 78.72296) (end 77.07704 79.5) (width 0.6) (layer "F.Cu") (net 1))
 (segment (start 77.722792 75.9) (end 76.3 77.322792) (width 0.6) (layer "F.Cu") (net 1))
 (segment (start 76.3 77.322792) (end 76.3 78.72296) (width 0.6) (layer "F.Cu") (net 1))
 (segment (start 95 91.31) (end 95 99) (width 0.6) (layer "F.Cu") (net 6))
 (segment (start 95 99) (end 95.5 99.5) (width 0.6) (layer "F.Cu") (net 6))
 (segment (start 89.15 86.65) (end 89.15 88.425) (width 0.6) (layer "F.Cu") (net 4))
 (segment (start 78.81 89.19) (end 82.152124 85.847876) (width 0.6) (layer "F.Cu") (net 4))
 (segment (start 89.15 88.425) (end 88.805 88.77) (width 0.6) (layer "F.Cu") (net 4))
 (segment (start 87.88 99.5) (end 86.43 100.95) (width 0.6) (layer "F.Cu") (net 4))
 (segment (start 82.879248 86.575) (end 89.075 86.575) (width 0.6) (layer "F.Cu") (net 4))
 (segment (start 88.805 88.77) (end 87.7 88.77) (width 0.6) (layer "F.Cu") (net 4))
 (segment (start 74.5 78.195752) (end 82.152124 85.847876) (width 0.6) (layer "F.Cu") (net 4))
 (segment (start 78.81 100.31) (end 78.81 89.19) (width 0.6) (layer "F.Cu") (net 4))
 (segment (start 74.5 77.35) (end 75 77.35) (width 0.6) (layer "F.Cu") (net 4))
 (segment (start 89.075 86.575) (end 89.15 86.65) (width 0.6) (layer "F.Cu") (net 4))
 (segment (start 82.152124 85.847876) (end 82.879248 86.575) (width 0.6) (layer "F.Cu") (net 4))
 (segment (start 86.43 100.95) (end 79.45 100.95) (width 0.6) (layer "F.Cu") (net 4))
 (segment (start 74.5 77.35) (end 74.5 78.195752) (width 0.6) (layer "F.Cu") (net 4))
 (segment (start 79.45 100.95) (end 78.81 100.31) (width 0.6) (layer "F.Cu") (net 4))
 (segment (start 74.49099 77.35) (end 74.5 77.35) (width 0.6) (layer "F.Cu") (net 4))
 (segment (start 90.42 91.9) (end 90.42 99.5) (width 0.6) (layer "F.Cu") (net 8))
 (segment (start 93.55 88.77) (end 90.42 91.9) (width 0.6) (layer "F.Cu") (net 8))
 (segment (start 95 88.77) (end 93.55 88.77) (width 0.6) (layer "F.Cu") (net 8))
 (segment (start 82.8 91.295) (end 82.8 99.5) (width 0.6) (layer "F.Cu") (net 3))
 (segment (start 87.7 87.5) (end 86.595 87.5) (width 0.6) (layer "F.Cu") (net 3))
 (segment (start 86.595 87.5) (end 82.8 91.295) (width 0.6) (layer "F.Cu") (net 3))
 (segment (start 90.5 88.347792) (end 90.5 82.15) (width 0.6) (layer "F.Cu") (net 5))
 (segment (start 86.595 90.04) (end 85.34 91.295) (width 0.6) (layer "F.Cu") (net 5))
 (segment (start 85.34 91.295) (end 85.34 99.5) (width 0.6) (layer "F.Cu") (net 5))
 (segment (start 88.807792 90.04) (end 90.5 88.347792) (width 0.6) (layer "F.Cu") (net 5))
 (segment (start 90.5 82.15) (end 84.2 75.85) (width 0.6) (layer "F.Cu") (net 5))
 (segment (start 87.7 90.04) (end 88.807792 90.04) (width 0.6) (layer "F.Cu") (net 5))
 (segment (start 84.2 75.85) (end 83.5 75.85) (width 0.6) (layer "F.Cu") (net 5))
 (segment (start 87.7 90.04) (end 86.595 90.04) (width 0.6) (layer "F.Cu") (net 5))
 (segment (start 80.26 99.5) (end 80.5 99.5) (width 0.6) (layer "F.Cu") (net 14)))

